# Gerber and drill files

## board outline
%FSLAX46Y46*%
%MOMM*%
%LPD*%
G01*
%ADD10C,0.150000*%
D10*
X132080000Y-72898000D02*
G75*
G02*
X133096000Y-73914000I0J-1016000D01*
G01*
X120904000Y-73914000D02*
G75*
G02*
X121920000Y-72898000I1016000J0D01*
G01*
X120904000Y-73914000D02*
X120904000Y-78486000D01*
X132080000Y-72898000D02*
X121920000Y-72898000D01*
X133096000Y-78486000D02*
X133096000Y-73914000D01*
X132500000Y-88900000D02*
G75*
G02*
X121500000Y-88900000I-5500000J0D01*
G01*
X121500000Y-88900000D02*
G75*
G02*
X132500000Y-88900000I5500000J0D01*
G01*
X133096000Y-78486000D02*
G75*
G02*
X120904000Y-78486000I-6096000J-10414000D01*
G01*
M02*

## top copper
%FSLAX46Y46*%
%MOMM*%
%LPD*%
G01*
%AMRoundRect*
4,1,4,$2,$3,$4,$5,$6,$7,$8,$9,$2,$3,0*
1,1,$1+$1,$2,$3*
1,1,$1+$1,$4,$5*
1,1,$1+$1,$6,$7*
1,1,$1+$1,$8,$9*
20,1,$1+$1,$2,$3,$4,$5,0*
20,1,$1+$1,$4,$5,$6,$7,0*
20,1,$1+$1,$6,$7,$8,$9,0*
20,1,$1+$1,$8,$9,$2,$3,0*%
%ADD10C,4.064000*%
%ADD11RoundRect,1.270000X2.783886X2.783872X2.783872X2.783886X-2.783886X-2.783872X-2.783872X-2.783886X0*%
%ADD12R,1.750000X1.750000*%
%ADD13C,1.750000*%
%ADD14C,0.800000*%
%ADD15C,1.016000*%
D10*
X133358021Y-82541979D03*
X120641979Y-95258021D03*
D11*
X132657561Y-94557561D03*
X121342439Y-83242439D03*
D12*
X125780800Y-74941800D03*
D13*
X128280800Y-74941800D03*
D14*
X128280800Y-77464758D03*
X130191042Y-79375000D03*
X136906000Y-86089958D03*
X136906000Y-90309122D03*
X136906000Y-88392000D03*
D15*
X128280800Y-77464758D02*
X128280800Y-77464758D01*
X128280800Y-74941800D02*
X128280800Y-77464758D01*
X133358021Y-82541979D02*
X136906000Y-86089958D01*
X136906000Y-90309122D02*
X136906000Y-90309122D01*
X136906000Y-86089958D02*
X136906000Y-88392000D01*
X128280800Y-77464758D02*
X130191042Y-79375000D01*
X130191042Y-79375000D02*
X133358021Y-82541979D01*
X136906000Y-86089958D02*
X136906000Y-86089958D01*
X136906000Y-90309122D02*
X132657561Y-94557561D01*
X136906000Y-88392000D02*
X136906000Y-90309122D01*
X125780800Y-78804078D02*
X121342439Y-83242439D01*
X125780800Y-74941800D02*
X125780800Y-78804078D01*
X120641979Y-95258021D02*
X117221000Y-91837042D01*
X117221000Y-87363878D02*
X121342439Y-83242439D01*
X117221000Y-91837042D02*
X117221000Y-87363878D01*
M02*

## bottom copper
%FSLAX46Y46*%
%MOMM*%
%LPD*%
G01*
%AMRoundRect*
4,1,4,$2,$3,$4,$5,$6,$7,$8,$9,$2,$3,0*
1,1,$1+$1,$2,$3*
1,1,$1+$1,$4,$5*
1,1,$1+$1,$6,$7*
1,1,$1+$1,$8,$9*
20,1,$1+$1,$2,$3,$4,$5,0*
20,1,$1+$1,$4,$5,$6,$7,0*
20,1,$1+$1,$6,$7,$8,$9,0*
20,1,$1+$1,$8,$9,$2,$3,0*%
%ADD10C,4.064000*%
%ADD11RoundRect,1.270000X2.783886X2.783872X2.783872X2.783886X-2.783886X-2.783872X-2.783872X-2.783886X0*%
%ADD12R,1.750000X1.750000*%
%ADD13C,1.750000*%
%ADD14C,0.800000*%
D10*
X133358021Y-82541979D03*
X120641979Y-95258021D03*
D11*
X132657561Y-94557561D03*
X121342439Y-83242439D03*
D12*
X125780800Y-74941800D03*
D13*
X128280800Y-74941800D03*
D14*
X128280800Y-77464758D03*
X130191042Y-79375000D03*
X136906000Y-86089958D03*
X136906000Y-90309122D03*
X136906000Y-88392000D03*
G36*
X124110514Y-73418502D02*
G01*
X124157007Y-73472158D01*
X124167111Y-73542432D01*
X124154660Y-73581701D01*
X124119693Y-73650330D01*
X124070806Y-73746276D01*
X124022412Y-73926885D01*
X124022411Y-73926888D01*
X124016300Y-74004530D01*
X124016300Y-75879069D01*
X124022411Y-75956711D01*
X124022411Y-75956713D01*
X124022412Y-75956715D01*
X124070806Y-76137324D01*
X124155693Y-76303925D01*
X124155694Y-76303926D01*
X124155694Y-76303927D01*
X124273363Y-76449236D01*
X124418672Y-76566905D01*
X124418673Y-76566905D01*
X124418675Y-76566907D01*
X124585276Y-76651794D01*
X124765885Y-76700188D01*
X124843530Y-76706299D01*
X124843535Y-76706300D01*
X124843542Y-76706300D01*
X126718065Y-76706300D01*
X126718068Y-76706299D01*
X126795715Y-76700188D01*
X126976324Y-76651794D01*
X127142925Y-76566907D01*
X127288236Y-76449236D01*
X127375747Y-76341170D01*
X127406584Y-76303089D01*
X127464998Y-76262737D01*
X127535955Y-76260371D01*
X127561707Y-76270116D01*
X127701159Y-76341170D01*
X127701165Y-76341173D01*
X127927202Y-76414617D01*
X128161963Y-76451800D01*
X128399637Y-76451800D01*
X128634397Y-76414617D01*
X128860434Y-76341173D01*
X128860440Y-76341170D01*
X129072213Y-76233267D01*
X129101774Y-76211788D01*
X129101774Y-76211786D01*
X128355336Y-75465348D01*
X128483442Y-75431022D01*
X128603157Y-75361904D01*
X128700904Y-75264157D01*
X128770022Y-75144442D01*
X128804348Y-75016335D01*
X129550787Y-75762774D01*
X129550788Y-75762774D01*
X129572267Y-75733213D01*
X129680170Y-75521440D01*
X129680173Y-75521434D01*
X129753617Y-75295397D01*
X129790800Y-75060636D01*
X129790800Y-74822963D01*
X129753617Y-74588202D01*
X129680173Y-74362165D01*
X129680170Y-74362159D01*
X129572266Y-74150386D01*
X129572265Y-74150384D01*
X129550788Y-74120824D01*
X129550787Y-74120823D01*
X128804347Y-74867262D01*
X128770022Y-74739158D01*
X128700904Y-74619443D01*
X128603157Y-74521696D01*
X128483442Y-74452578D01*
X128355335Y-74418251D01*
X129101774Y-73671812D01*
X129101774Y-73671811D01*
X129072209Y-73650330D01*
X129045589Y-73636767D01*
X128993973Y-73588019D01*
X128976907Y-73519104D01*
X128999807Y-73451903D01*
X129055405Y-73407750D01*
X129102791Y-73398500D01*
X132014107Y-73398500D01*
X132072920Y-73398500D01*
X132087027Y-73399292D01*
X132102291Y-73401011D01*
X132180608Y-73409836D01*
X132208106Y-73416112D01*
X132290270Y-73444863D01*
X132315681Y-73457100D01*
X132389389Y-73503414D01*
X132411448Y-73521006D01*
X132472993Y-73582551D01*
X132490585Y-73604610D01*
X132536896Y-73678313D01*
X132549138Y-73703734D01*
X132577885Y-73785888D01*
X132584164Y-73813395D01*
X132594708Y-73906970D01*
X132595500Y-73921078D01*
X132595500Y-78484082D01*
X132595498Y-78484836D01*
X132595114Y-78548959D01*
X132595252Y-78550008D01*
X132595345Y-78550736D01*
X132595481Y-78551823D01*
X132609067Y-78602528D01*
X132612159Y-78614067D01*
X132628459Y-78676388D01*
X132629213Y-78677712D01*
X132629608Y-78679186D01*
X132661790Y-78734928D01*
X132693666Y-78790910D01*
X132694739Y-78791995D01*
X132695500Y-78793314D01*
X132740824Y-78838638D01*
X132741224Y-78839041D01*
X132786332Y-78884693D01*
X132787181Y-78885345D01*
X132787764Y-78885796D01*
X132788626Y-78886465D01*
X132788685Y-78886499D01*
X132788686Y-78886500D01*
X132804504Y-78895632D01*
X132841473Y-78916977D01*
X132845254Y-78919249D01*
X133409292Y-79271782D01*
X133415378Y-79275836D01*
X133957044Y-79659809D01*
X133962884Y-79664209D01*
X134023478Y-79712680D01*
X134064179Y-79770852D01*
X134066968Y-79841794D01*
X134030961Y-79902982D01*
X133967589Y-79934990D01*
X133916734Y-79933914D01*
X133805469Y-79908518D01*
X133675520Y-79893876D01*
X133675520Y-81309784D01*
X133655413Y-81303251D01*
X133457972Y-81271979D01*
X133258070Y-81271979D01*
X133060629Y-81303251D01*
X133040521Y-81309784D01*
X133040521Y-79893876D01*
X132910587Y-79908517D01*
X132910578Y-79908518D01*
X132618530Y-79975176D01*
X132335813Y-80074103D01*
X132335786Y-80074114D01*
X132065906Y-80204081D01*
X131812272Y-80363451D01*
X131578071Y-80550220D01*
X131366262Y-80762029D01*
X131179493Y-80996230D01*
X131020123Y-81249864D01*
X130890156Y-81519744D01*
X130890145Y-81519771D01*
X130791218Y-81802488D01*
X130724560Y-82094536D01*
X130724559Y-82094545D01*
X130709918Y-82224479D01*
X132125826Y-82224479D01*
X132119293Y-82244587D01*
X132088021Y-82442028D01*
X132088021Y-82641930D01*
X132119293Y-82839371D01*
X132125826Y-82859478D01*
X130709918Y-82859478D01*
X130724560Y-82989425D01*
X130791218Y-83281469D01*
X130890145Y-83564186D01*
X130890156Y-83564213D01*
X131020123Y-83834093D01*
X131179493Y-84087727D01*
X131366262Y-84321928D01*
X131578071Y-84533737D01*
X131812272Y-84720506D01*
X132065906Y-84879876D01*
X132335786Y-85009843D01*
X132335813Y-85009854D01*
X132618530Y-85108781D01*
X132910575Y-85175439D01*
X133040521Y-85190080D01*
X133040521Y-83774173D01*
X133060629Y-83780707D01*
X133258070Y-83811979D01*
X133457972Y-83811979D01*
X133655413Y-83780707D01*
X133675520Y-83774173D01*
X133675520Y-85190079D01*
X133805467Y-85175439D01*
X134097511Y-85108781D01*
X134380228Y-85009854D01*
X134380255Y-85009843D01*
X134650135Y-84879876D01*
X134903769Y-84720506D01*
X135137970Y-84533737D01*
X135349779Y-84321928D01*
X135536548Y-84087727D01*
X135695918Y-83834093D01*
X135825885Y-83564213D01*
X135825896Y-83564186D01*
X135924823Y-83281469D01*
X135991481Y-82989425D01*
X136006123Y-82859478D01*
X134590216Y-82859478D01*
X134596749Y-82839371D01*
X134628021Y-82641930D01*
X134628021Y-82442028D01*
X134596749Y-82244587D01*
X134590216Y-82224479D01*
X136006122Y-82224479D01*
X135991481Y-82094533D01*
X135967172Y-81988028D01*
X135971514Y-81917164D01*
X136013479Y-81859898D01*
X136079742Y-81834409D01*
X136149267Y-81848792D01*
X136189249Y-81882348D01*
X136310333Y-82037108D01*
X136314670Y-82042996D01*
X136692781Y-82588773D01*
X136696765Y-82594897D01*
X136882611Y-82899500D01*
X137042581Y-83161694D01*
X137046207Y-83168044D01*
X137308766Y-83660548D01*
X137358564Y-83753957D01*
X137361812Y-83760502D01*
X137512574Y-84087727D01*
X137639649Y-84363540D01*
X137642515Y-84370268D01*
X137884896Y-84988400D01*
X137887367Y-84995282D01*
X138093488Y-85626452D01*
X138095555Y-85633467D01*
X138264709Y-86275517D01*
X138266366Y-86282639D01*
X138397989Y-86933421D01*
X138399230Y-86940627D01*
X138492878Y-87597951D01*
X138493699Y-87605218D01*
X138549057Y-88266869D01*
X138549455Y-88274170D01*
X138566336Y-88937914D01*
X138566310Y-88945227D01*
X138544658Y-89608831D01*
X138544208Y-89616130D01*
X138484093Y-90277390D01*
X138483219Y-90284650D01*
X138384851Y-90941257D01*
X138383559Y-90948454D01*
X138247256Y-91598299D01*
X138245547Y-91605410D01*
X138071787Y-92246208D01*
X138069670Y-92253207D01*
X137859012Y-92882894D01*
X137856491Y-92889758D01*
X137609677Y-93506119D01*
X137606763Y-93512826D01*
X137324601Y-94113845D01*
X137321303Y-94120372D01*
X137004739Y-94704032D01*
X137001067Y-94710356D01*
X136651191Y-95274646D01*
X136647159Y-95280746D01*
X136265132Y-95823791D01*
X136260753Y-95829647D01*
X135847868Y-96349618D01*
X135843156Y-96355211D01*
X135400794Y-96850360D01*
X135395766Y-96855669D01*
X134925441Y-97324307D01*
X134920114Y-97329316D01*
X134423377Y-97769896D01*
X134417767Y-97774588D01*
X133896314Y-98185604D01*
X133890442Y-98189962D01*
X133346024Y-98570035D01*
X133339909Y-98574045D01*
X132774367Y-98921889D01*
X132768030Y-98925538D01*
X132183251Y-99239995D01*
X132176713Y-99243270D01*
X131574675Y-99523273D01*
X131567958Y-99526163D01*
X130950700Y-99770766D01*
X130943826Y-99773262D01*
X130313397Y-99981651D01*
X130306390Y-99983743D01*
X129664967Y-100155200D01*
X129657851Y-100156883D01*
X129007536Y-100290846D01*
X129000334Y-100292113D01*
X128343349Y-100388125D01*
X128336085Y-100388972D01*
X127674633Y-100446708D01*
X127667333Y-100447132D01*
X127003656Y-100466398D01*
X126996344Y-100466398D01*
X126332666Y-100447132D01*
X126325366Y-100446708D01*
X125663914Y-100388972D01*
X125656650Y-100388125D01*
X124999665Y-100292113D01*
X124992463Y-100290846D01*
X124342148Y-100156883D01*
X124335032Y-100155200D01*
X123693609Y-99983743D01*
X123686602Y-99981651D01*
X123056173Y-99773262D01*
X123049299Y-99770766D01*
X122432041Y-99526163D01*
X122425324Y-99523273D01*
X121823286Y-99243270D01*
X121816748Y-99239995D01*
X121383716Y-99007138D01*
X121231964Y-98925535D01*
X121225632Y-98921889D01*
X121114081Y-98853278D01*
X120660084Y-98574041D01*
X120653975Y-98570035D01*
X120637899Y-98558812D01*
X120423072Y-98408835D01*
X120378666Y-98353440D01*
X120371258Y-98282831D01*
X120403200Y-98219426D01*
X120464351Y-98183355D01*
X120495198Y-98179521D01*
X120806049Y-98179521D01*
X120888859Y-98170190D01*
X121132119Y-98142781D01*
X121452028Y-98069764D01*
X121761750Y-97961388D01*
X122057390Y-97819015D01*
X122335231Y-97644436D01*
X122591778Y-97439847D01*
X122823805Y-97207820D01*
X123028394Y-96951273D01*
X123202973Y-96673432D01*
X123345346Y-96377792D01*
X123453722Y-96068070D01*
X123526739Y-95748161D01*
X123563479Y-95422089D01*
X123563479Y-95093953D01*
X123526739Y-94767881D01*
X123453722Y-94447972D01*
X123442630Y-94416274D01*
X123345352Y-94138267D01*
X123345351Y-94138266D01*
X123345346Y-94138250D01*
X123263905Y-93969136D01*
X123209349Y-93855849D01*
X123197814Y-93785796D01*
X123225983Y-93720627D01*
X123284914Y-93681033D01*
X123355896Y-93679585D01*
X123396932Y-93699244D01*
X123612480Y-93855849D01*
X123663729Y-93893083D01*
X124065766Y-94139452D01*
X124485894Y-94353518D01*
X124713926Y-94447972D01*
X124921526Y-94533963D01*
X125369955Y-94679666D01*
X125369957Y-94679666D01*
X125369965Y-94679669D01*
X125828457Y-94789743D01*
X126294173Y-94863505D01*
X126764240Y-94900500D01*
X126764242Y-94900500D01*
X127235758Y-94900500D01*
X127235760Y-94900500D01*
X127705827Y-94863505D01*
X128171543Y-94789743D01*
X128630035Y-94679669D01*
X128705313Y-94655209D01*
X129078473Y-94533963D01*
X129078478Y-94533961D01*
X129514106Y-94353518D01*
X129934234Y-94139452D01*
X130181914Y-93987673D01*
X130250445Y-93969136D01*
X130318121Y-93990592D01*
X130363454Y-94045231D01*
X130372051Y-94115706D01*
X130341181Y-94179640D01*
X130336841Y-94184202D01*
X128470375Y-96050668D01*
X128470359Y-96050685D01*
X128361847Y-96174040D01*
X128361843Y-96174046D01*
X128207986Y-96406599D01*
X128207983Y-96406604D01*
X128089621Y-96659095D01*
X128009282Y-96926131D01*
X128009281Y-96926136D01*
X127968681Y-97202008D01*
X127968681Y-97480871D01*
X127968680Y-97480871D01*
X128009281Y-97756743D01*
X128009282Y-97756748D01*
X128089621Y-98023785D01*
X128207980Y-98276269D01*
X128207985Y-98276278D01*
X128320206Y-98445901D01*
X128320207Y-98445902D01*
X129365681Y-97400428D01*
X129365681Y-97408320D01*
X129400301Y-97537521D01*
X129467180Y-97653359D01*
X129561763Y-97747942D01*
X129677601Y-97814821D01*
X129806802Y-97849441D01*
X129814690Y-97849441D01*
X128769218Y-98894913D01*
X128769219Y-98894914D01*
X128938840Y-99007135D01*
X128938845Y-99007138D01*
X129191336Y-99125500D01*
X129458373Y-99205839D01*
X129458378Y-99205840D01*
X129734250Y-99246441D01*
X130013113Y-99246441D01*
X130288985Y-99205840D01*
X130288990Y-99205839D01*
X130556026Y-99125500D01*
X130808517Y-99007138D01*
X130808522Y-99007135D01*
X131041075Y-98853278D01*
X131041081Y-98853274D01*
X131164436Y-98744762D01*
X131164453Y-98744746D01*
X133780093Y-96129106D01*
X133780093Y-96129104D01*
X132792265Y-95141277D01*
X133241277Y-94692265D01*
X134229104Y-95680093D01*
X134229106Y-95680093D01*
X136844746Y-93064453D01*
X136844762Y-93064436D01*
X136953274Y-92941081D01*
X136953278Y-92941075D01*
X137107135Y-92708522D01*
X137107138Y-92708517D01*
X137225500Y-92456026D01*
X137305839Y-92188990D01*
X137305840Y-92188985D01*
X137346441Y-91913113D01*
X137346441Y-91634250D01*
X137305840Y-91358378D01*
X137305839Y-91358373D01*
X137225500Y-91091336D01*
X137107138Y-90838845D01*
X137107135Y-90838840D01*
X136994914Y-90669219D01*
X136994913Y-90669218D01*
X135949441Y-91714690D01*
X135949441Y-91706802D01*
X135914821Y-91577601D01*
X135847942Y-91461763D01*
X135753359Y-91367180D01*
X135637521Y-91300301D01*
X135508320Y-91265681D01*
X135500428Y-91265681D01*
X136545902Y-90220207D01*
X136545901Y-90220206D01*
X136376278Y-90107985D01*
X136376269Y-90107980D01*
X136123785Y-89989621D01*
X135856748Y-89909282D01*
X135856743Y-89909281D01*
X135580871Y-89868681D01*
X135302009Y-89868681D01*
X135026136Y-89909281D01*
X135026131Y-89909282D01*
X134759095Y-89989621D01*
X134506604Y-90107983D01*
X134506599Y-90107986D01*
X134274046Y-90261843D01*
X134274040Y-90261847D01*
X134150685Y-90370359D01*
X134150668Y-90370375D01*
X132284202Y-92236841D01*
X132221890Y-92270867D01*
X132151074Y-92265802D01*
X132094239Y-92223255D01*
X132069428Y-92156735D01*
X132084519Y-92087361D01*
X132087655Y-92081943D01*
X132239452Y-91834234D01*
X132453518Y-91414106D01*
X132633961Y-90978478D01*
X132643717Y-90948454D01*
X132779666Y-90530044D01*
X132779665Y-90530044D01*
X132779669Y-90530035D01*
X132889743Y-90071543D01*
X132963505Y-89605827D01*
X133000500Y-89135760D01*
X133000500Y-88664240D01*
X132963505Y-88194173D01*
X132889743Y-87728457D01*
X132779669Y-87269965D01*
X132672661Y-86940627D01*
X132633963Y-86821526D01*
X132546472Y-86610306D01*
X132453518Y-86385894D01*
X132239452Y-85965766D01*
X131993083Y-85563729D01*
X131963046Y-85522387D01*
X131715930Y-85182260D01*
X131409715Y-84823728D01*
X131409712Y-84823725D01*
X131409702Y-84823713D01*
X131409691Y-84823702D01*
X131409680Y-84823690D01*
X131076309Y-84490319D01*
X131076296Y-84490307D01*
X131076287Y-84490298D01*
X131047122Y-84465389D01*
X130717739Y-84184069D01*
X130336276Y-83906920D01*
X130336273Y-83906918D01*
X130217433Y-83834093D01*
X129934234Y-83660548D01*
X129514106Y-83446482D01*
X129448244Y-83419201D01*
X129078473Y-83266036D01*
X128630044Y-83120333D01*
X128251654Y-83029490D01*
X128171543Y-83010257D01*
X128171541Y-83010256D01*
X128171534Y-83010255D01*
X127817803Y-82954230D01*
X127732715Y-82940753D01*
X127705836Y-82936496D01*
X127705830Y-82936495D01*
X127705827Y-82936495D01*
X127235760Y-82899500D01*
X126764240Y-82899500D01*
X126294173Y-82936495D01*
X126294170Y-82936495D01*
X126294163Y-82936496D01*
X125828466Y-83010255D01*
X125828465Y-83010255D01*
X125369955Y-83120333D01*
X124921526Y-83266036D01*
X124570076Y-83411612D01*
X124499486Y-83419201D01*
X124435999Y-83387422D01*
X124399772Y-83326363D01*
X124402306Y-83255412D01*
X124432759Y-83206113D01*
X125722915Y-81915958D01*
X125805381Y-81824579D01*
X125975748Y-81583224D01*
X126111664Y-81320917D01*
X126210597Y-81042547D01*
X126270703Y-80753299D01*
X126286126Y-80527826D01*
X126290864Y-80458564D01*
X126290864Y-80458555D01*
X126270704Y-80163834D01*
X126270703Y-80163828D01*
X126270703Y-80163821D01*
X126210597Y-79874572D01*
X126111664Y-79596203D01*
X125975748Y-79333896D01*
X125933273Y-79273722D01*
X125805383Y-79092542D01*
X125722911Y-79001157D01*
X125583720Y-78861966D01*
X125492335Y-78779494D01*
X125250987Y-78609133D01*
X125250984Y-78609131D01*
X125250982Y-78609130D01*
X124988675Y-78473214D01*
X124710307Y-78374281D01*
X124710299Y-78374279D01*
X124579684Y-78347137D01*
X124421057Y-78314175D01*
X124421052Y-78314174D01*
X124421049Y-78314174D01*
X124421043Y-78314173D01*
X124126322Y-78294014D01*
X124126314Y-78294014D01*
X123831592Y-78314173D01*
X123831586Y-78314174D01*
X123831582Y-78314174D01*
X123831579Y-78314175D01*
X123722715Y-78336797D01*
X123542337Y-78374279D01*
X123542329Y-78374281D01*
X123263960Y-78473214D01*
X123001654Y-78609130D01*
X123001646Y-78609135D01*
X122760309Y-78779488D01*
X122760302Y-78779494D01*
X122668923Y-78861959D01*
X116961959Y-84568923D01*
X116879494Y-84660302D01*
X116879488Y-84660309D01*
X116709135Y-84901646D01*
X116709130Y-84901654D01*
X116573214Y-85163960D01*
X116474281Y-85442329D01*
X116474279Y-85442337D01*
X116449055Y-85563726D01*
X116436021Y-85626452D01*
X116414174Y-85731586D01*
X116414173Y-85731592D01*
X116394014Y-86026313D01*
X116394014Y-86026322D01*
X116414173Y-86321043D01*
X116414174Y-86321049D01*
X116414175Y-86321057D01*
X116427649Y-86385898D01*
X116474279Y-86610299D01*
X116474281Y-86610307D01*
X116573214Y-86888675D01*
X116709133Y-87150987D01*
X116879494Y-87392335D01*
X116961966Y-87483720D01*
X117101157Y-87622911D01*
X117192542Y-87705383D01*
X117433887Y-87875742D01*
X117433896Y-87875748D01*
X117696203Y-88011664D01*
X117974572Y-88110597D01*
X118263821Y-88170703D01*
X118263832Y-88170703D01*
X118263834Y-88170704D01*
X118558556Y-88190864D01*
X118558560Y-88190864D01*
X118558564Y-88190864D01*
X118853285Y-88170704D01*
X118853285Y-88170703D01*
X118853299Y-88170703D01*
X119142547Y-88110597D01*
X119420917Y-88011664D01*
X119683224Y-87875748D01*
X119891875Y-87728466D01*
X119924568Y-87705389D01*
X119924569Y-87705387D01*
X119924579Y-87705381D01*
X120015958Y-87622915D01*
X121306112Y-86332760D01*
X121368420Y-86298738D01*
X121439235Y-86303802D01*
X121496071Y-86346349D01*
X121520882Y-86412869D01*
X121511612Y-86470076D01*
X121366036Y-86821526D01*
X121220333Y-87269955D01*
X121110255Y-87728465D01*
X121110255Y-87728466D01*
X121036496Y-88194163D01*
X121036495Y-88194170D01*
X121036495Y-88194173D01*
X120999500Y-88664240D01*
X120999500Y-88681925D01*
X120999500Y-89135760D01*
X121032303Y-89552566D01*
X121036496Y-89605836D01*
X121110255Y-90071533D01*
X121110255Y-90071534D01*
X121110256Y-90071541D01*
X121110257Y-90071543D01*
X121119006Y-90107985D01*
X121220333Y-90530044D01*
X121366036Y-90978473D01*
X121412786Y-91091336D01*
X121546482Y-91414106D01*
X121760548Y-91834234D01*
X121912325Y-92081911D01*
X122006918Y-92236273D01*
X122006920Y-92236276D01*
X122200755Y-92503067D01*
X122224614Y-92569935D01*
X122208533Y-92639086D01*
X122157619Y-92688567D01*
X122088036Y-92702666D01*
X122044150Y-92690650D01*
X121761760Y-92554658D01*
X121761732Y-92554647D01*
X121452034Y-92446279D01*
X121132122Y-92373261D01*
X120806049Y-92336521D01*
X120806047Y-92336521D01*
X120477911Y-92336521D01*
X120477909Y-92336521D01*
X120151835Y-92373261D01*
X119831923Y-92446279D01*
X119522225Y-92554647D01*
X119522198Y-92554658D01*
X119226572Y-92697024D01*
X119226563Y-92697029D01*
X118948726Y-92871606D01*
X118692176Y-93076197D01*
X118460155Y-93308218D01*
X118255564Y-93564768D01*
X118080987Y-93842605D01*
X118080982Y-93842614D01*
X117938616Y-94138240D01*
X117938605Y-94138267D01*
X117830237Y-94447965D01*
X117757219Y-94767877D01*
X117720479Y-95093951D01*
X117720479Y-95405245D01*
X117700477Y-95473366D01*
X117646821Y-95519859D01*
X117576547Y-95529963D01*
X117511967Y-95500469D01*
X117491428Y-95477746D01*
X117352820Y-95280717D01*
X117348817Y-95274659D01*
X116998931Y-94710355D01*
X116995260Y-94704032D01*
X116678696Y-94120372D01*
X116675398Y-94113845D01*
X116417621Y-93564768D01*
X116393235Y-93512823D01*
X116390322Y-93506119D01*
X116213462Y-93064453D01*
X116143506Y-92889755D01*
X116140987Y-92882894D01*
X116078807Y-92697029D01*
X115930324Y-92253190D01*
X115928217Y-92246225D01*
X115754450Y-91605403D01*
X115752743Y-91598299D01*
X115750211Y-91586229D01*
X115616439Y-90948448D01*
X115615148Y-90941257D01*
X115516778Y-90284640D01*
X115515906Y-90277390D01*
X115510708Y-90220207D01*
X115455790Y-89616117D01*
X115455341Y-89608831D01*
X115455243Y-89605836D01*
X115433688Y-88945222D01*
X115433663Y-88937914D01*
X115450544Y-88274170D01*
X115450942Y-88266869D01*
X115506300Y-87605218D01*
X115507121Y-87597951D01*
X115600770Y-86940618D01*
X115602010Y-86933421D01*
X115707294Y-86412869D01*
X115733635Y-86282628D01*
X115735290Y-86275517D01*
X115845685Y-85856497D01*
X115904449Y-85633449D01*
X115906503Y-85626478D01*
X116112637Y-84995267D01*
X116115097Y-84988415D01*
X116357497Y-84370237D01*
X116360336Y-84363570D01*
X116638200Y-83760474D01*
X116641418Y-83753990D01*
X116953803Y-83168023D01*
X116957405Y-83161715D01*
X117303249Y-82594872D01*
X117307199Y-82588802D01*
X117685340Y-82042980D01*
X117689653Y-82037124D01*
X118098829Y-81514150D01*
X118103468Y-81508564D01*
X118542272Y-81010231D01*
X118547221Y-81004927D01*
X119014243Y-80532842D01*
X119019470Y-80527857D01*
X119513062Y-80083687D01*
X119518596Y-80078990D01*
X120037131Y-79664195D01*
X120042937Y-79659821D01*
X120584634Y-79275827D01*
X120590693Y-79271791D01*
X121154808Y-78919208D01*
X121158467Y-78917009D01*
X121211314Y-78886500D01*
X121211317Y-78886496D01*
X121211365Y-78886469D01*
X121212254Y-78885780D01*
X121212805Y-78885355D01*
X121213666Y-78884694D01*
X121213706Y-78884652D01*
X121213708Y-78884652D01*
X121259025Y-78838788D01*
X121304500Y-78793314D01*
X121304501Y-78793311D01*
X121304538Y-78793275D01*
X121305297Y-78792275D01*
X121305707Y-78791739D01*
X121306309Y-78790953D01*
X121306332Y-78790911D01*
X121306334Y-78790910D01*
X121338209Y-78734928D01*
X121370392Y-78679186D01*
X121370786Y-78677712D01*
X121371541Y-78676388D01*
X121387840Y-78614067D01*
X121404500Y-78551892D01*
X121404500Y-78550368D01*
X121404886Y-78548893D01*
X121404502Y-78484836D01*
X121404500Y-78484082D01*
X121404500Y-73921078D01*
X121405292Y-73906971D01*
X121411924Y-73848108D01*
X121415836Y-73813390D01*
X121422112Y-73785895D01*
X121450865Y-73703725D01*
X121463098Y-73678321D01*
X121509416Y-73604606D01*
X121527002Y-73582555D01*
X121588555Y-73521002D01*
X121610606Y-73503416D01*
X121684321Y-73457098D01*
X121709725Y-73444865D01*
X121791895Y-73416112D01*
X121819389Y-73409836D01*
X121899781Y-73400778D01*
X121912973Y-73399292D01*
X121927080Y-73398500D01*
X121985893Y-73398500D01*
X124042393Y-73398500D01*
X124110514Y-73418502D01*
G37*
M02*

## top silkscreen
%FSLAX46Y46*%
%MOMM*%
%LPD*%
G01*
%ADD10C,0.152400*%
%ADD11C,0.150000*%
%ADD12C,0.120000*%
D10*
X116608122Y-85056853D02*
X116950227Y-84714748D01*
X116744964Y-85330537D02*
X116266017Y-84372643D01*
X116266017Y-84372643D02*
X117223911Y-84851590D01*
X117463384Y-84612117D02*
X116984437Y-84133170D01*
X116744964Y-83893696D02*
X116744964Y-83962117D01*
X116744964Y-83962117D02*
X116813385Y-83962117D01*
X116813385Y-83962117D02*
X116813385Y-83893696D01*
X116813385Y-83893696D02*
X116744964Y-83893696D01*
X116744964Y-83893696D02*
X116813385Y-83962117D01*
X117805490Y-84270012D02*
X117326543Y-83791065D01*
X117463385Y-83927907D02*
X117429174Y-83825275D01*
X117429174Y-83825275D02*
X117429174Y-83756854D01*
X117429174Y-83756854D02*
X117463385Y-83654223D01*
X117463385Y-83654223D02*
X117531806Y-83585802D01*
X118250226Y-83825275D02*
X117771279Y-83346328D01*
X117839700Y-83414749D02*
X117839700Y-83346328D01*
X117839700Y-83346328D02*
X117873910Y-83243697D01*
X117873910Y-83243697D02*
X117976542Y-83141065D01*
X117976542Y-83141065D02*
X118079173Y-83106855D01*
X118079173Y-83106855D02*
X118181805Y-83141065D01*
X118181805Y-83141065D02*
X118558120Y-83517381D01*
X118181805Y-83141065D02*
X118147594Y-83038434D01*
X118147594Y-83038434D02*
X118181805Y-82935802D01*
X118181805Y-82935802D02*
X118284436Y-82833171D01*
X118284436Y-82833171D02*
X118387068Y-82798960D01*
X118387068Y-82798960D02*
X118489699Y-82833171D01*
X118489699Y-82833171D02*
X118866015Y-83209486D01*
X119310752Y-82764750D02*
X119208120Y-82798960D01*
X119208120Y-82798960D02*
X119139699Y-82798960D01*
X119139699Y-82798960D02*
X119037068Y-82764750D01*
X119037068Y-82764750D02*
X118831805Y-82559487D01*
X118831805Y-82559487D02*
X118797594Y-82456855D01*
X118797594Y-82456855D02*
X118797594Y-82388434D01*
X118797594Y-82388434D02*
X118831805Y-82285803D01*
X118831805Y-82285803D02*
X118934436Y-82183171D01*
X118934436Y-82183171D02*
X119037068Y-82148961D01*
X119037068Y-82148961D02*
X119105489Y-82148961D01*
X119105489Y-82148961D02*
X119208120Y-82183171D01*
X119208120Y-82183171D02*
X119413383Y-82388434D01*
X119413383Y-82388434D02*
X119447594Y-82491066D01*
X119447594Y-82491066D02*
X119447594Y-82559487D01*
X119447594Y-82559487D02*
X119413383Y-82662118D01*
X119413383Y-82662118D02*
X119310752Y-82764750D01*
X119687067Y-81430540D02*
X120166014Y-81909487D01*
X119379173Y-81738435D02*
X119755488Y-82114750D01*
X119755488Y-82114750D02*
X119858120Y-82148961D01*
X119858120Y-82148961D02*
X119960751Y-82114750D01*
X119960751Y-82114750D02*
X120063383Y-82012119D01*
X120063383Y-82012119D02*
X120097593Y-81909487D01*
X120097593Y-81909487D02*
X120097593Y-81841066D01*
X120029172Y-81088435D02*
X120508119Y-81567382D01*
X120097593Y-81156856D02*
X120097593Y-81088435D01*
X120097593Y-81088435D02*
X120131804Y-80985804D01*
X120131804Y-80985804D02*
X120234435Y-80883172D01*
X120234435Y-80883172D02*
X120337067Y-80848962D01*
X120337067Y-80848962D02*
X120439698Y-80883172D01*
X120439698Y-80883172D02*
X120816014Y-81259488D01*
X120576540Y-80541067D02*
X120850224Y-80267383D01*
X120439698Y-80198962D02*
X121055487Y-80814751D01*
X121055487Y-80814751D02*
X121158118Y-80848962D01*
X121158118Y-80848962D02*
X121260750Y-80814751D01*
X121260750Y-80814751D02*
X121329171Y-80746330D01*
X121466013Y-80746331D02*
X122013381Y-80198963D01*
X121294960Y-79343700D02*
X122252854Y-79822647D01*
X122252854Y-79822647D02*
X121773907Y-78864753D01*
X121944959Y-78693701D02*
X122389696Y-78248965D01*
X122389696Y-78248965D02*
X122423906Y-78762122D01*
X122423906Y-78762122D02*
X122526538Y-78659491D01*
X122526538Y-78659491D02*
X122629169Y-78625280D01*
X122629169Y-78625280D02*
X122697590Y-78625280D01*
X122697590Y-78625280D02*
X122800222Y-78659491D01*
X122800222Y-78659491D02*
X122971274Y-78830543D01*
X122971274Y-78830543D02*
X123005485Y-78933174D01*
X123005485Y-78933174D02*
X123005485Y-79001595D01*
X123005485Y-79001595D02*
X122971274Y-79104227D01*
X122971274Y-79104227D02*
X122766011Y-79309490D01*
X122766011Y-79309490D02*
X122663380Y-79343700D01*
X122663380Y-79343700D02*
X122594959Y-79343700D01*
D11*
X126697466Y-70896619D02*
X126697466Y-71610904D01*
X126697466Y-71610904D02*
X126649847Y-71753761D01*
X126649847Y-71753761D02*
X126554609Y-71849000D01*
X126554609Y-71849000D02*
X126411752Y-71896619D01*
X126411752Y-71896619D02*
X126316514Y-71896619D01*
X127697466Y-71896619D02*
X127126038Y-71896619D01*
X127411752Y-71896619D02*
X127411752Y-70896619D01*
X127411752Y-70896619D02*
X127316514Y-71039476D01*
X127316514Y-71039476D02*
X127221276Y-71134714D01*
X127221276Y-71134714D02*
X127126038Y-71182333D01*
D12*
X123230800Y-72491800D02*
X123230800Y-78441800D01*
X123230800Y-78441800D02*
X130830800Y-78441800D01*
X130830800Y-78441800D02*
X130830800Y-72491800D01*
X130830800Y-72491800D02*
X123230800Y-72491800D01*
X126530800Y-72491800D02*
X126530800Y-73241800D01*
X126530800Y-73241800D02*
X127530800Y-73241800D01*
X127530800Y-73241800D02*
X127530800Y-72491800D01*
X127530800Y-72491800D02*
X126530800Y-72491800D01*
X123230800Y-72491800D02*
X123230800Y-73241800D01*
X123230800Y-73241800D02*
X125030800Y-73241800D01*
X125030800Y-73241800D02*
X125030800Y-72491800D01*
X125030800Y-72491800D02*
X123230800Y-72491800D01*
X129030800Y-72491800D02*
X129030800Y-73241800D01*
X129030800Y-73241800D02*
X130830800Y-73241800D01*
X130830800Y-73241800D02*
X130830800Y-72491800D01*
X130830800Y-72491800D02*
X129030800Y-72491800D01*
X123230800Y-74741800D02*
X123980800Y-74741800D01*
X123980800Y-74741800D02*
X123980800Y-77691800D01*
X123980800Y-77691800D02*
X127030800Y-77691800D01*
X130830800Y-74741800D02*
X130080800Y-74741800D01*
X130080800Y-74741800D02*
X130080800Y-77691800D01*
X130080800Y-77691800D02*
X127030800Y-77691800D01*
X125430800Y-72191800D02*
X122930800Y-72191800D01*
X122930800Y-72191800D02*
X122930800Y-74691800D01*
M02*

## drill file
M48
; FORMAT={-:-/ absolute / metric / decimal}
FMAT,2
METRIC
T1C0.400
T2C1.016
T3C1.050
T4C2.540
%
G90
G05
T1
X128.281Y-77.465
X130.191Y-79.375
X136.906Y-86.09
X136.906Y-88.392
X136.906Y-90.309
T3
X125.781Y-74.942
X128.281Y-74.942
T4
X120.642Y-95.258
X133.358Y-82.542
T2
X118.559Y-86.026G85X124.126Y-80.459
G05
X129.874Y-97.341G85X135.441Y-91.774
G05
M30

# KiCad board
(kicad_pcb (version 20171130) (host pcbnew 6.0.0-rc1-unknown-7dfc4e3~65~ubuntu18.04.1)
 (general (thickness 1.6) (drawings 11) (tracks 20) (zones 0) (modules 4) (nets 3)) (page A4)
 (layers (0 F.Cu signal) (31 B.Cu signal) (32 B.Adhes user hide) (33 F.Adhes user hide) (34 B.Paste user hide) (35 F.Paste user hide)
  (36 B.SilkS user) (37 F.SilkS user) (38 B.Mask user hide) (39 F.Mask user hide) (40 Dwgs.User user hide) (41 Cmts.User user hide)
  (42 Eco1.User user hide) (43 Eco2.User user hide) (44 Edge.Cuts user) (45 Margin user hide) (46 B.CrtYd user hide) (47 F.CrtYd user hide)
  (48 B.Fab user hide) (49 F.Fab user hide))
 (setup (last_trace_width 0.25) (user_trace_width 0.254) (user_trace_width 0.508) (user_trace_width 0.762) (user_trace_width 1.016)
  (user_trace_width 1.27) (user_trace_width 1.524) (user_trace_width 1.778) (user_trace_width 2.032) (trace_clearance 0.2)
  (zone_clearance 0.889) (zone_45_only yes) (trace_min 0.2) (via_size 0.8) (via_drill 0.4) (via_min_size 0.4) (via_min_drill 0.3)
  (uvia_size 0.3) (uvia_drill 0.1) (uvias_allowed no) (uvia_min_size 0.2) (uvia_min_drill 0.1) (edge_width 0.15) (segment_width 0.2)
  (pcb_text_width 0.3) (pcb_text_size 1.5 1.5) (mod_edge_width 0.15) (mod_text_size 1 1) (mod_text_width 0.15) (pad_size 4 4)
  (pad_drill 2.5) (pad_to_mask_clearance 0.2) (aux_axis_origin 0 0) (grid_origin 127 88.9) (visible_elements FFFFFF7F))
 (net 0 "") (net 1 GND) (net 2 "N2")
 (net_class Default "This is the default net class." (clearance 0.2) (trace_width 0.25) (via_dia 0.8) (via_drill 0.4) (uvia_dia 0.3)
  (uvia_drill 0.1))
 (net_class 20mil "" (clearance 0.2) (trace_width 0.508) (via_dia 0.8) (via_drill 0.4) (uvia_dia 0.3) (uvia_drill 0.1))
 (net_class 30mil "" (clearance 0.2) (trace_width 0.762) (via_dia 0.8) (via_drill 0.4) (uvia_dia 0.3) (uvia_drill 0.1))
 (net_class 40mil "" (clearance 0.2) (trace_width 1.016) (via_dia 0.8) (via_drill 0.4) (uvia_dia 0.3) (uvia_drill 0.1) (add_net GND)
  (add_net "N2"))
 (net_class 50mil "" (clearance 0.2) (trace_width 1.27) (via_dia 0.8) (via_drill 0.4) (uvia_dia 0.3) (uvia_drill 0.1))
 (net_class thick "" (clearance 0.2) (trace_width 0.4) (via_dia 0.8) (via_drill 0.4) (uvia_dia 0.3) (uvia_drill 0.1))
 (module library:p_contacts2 (layer F.Cu) (at 127 88.9 45)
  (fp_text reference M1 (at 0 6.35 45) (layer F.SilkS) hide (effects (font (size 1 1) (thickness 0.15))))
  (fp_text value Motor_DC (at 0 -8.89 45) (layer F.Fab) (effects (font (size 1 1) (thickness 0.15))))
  (pad 2 thru_hole circle (at 8.9916 0 45) (size 4.064 4.064) (drill 2.54) (layers *.Mask F.Cu) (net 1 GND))
  (pad 1 thru_hole circle (at -8.9916 0 45) (size 4.064 4.064) (drill 2.54) (layers *.Mask F.Cu) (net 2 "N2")))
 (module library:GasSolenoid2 (layer F.Cu) (at 127 88.9 135)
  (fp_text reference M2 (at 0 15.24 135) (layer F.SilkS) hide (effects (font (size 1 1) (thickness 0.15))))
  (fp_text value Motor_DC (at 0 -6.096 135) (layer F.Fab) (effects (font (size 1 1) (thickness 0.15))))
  (pad 2 thru_hole roundrect (at -8.000999 0 135) (size 2.54 10.414) (drill oval 1.016 8.89) (layers *.Mask F.Cu) (roundrect_rratio 0.5)
   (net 1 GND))
  (pad 1 thru_hole roundrect (at 8.000999 0 135) (size 2.54 10.414) (drill oval 1.016 8.89) (layers *.Mask F.Cu) (roundrect_rratio 0.5)
   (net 2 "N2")))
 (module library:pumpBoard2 (layer F.Cu) (at 127 88.9)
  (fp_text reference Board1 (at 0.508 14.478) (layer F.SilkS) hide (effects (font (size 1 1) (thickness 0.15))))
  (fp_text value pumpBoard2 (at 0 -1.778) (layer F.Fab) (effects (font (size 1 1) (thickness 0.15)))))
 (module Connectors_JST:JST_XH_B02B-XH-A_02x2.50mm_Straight (layer F.Cu) (at 125.7808 74.9418)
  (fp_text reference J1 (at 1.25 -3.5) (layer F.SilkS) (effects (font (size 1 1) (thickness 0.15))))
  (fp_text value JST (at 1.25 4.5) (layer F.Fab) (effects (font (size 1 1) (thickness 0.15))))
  (fp_line (start -2.55 -2.45) (end -2.55 3.5) (layer F.SilkS) (width 0.12))
  (fp_line (start -2.55 3.5) (end 5.05 3.5) (layer F.SilkS) (width 0.12))
  (fp_line (start 5.05 3.5) (end 5.05 -2.45) (layer F.SilkS) (width 0.12))
  (fp_line (start 5.05 -2.45) (end -2.55 -2.45) (layer F.SilkS) (width 0.12))
  (fp_line (start 0.75 -2.45) (end 0.75 -1.7) (layer F.SilkS) (width 0.12))
  (fp_line (start 0.75 -1.7) (end 1.75 -1.7) (layer F.SilkS) (width 0.12))
  (fp_line (start 1.75 -1.7) (end 1.75 -2.45) (layer F.SilkS) (width 0.12))
  (fp_line (start 1.75 -2.45) (end 0.75 -2.45) (layer F.SilkS) (width 0.12))
  (fp_line (start -2.55 -2.45) (end -2.55 -1.7) (layer F.SilkS) (width 0.12))
  (fp_line (start -2.55 -1.7) (end -0.75 -1.7) (layer F.SilkS) (width 0.12))
  (fp_line (start -0.75 -1.7) (end -0.75 -2.45) (layer F.SilkS) (width 0.12))
  (fp_line (start -0.75 -2.45) (end -2.55 -2.45) (layer F.SilkS) (width 0.12))
  (fp_line (start 3.25 -2.45) (end 3.25 -1.7) (layer F.SilkS) (width 0.12))
  (fp_line (start 3.25 -1.7) (end 5.05 -1.7) (layer F.SilkS) (width 0.12))
  (fp_line (start 5.05 -1.7) (end 5.05 -2.45) (layer F.SilkS) (width 0.12))
  (fp_line (start 5.05 -2.45) (end 3.25 -2.45) (layer F.SilkS) (width 0.12))
  (fp_line (start -2.55 -0.2) (end -1.8 -0.2) (layer F.SilkS) (width 0.12))
  (fp_line (start -1.8 -0.2) (end -1.8 2.75) (layer F.SilkS) (width 0.12))
  (fp_line (start -1.8 2.75) (end 1.25 2.75) (layer F.SilkS) (width 0.12))
  (fp_line (start 5.05 -0.2) (end 4.3 -0.2) (layer F.SilkS) (width 0.12))
  (fp_line (start 4.3 -0.2) (end 4.3 2.75) (layer F.SilkS) (width 0.12))
  (fp_line (start 4.3 2.75) (end 1.25 2.75) (layer F.SilkS) (width 0.12))
  (fp_line (start -0.35 -2.75) (end -2.85 -2.75) (layer F.SilkS) (width 0.12))
  (fp_line (start -2.85 -2.75) (end -2.85 -0.25) (layer F.SilkS) (width 0.12))
  (pad 1 thru_hole rect (at 0 0) (size 1.75 1.75) (drill 1.05) (layers *.Cu *.Mask) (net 2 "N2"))
  (pad 2 thru_hole circle (at 2.5 0) (size 1.75 1.75) (drill 1.05) (layers *.Cu *.Mask) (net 1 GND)))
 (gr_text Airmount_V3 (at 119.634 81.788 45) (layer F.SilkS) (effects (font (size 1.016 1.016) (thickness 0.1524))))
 (gr_arc (start 132.08 73.914) (end 133.096 73.914) (angle -90) (layer Edge.Cuts) (width 0.15))
 (gr_arc (start 121.92 73.914) (end 121.92 72.898) (angle -90) (layer Edge.Cuts) (width 0.15))
 (gr_line (start 120.904 73.914) (end 120.904 78.486) (layer Edge.Cuts) (width 0.15))
 (gr_line (start 132.08 72.898) (end 121.92 72.898) (layer Edge.Cuts) (width 0.15))
 (gr_line (start 133.096 78.486) (end 133.096 73.914) (layer Edge.Cuts) (width 0.15))
 (gr_circle (center 127 88.9) (end 132.5 88.9) (layer Edge.Cuts) (width 0.15))
 (gr_arc (start 127 88.9) (end 120.904 78.486) (angle -299.3135022) (layer Edge.Cuts) (width 0.15))
 (segment (start 128.2808 77.464758) (end 128.2808 77.464758) (width 1.016) (layer F.Cu) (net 1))
 (segment (start 128.2808 74.9418) (end 128.2808 77.464758) (width 1.016) (layer F.Cu) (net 1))
 (segment (start 133.358021 82.541979) (end 136.906 86.089958) (width 1.016) (layer F.Cu) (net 1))
 (segment (start 136.906 90.309122) (end 136.906 90.309122) (width 1.016) (layer F.Cu) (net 1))
 (segment (start 136.906 86.089958) (end 136.906 88.392) (width 1.016) (layer F.Cu) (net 1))
 (segment (start 128.2808 77.464758) (end 130.191042 79.375) (width 1.016) (layer F.Cu) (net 1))
 (via (at 128.2808 77.464758) (size 0.8) (drill 0.4) (layers F.Cu B.Cu) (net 1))
 (segment (start 130.191042 79.375) (end 133.358021 82.541979) (width 1.016) (layer F.Cu) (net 1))
 (via (at 130.191042 79.375) (size 0.8) (drill 0.4) (layers F.Cu B.Cu) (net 1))
 (segment (start 136.906 86.089958) (end 136.906 86.089958) (width 1.016) (layer F.Cu) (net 1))
 (via (at 136.906 86.089958) (size 0.8) (drill 0.4) (layers F.Cu B.Cu) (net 1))
 (segment (start 136.906 90.309122) (end 132.657561 94.557561) (width 1.016) (layer F.Cu) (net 1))
 (via (at 136.906 90.309122) (size 0.8) (drill 0.4) (layers F.Cu B.Cu) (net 1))
 (segment (start 136.906 88.392) (end 136.906 90.309122) (width 1.016) (layer F.Cu) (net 1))
 (via (at 136.906 88.392) (size 0.8) (drill 0.4) (layers F.Cu B.Cu) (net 1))
 (segment (start 125.7808 78.804078) (end 121.342439 83.242439) (width 1.016) (layer F.Cu) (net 2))
 (segment (start 125.7808 74.9418) (end 125.7808 78.804078) (width 1.016) (layer F.Cu) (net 2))
 (segment (start 120.641979 95.258021) (end 117.221 91.837042) (width 1.016) (layer F.Cu) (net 2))
 (segment (start 117.221 87.363878) (end 121.342439 83.242439) (width 1.016) (layer F.Cu) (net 2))
 (segment (start 117.221 91.837042) (end 117.221 87.363878) (width 1.016) (layer F.Cu) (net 2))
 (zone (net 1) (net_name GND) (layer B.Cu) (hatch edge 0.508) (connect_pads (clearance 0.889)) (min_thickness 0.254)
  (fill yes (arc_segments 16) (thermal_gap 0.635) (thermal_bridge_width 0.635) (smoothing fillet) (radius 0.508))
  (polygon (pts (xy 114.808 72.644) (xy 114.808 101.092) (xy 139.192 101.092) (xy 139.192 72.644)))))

